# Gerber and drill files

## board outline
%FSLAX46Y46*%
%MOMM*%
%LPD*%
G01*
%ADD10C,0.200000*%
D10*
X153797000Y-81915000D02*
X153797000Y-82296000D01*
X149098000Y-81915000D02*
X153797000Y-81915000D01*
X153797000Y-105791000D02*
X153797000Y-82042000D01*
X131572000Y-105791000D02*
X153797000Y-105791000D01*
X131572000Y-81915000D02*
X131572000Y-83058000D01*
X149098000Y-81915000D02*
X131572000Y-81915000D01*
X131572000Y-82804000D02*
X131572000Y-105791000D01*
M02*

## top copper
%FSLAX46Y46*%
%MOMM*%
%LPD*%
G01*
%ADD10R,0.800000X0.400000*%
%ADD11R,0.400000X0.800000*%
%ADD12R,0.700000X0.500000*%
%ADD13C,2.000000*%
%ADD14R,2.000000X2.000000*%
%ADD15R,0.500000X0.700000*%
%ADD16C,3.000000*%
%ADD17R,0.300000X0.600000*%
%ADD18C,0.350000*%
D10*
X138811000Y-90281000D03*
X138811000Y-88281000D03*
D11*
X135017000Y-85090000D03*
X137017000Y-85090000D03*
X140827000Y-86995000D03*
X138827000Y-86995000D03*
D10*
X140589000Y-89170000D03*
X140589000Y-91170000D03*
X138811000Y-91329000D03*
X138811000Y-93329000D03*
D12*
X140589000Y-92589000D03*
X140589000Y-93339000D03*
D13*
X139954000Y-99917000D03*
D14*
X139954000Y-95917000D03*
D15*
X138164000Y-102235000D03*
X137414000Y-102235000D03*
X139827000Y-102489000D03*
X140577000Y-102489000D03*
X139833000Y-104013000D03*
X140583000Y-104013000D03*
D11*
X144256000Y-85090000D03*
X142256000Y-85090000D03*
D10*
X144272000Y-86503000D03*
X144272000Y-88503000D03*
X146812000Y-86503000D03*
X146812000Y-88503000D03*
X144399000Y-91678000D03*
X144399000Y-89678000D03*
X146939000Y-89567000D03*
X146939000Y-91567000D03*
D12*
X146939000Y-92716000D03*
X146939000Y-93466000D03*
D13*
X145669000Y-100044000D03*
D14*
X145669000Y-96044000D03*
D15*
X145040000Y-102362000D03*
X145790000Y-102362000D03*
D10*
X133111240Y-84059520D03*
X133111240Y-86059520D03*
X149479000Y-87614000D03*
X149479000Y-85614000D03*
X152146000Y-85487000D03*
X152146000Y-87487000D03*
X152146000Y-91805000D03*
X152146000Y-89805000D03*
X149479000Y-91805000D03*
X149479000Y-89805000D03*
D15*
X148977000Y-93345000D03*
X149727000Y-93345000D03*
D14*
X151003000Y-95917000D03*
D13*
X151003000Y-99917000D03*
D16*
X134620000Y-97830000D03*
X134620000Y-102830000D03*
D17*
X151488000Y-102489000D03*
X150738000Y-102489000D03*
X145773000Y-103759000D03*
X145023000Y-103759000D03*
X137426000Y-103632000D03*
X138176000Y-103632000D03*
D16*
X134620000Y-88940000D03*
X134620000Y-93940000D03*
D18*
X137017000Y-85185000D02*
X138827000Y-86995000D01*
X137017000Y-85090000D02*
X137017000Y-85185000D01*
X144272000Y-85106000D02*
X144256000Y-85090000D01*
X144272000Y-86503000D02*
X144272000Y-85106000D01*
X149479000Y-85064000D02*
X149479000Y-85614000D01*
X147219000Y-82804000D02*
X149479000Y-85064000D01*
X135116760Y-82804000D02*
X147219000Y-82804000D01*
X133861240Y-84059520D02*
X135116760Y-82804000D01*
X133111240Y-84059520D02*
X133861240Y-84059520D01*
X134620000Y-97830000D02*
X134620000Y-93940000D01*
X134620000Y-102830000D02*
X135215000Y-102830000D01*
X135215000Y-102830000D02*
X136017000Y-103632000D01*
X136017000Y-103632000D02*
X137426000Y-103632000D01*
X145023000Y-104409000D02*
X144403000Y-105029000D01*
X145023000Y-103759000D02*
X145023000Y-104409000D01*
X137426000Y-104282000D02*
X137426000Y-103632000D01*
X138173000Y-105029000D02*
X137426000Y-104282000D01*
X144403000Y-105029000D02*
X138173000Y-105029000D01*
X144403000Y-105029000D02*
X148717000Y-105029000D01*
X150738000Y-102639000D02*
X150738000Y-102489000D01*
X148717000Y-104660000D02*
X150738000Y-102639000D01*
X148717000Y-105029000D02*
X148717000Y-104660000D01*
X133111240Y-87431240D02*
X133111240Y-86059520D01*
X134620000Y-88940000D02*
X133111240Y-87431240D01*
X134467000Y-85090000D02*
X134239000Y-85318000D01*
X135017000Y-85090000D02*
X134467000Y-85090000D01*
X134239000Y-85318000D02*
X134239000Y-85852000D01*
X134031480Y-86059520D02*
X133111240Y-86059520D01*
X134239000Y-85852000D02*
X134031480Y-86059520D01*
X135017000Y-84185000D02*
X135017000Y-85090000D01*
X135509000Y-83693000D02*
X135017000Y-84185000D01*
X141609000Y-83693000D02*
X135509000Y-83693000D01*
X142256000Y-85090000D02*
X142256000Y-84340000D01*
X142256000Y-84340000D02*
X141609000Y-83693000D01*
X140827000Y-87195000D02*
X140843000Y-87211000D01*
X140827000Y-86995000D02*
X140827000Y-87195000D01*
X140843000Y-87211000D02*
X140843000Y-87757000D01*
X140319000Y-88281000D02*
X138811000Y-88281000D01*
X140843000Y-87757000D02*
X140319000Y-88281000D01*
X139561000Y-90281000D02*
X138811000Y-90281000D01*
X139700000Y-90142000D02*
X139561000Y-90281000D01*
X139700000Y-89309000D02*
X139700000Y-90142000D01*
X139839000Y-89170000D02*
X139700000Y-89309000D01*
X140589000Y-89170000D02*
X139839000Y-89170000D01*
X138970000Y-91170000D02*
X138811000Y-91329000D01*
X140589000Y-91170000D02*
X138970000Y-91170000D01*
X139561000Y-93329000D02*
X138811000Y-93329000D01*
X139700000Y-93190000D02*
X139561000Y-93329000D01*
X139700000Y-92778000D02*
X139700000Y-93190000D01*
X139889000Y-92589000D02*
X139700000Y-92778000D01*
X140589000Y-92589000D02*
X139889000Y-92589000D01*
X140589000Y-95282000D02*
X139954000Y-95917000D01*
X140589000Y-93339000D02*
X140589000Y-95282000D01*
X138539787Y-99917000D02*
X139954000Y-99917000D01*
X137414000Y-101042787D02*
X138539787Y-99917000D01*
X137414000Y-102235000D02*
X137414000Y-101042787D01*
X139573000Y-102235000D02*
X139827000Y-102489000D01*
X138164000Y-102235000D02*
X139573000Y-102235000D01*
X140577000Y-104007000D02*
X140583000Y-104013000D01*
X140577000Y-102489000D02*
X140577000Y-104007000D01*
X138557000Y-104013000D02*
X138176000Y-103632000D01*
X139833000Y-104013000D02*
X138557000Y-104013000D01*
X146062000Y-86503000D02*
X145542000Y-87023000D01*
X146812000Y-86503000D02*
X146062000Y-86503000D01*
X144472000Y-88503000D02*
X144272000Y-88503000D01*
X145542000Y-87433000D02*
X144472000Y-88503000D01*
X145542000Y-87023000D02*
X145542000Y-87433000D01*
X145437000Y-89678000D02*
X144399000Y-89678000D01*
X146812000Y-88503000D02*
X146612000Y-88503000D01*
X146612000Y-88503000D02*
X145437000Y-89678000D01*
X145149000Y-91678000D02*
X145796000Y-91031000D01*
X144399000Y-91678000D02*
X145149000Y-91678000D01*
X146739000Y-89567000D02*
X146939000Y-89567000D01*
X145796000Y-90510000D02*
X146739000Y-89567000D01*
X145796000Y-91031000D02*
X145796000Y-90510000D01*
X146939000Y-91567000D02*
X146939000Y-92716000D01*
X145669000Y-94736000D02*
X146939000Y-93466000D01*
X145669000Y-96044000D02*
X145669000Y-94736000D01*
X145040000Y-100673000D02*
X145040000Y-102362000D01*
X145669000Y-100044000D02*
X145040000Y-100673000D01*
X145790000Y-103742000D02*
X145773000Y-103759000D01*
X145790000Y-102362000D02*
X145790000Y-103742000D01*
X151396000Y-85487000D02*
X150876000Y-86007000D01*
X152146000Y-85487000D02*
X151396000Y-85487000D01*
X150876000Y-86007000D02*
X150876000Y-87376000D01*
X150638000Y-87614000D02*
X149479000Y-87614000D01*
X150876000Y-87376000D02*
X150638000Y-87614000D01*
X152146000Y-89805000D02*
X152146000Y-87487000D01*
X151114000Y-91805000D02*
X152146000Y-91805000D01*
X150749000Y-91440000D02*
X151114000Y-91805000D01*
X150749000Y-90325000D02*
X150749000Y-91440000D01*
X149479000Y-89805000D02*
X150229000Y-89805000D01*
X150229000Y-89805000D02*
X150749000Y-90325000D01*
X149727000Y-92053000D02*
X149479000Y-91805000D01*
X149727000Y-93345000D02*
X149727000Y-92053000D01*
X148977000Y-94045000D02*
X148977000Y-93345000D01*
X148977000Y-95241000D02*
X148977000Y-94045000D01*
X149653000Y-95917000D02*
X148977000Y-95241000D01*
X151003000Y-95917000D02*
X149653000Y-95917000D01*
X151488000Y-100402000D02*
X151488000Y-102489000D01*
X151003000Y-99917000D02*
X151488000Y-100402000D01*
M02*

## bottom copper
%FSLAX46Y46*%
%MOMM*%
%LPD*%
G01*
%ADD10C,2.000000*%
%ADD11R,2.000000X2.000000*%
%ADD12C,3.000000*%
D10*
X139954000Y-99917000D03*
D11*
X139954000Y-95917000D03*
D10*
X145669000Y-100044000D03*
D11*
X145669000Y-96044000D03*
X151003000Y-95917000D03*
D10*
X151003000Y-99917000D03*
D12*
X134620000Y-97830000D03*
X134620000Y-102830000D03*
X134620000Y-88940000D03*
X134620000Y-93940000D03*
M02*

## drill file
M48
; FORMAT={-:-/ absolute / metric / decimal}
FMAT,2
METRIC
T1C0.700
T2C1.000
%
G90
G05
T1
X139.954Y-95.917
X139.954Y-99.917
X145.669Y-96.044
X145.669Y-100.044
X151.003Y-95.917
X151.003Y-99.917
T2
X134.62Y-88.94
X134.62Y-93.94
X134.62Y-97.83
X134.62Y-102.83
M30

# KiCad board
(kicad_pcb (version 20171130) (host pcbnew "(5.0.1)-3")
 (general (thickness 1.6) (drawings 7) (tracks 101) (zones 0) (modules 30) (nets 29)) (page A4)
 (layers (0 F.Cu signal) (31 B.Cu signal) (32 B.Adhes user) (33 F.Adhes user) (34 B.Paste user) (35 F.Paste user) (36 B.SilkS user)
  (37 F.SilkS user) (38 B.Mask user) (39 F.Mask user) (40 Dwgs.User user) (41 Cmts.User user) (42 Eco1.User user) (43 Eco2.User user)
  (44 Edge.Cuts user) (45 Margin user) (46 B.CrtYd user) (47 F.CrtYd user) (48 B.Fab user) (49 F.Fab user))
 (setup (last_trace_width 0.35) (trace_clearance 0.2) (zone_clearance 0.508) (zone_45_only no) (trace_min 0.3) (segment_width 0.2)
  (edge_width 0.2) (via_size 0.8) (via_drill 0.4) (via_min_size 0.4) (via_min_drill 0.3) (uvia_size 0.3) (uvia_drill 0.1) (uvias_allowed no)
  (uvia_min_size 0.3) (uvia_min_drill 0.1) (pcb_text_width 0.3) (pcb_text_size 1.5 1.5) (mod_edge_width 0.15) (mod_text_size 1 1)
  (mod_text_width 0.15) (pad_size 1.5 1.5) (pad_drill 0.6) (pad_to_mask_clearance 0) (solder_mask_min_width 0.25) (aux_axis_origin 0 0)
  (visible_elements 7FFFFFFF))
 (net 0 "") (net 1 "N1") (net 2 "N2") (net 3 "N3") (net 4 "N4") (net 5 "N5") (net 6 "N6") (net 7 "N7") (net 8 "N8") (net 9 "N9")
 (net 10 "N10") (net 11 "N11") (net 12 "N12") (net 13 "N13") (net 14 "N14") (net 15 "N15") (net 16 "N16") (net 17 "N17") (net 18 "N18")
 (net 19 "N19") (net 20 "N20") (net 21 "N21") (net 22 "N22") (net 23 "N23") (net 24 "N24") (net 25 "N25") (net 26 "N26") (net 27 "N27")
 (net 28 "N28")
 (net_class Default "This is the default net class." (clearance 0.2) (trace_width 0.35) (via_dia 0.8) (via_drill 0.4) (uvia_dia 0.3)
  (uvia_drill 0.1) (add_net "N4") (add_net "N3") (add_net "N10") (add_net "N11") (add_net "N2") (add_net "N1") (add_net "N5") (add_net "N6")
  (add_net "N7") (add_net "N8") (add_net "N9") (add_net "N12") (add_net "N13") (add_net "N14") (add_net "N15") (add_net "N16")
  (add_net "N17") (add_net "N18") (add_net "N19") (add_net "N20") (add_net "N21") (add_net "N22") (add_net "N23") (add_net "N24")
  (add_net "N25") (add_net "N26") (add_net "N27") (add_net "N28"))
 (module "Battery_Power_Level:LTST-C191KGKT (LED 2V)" (layer F.Cu) (at 138.811 89.281 180)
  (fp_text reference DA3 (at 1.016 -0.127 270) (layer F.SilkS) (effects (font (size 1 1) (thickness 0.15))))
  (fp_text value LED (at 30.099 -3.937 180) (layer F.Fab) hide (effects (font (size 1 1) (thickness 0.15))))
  (pad 1 smd rect (at 0 -1 180) (size 0.8 0.4) (layers F.Cu F.Paste F.Mask) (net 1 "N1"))
  (pad 2 smd rect (at 0 1 180) (size 0.8 0.4) (layers F.Cu F.Paste F.Mask) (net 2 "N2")))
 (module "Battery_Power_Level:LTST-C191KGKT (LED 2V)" (layer F.Cu) (at 136.017 85.09 270)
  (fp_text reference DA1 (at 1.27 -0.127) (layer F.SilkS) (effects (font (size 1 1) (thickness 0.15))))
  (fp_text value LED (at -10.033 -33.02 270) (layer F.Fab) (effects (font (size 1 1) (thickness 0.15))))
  (pad 2 smd rect (at 0 1 270) (size 0.8 0.4) (layers F.Cu F.Paste F.Mask) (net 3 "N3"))
  (pad 1 smd rect (at 0 -1 270) (size 0.8 0.4) (layers F.Cu F.Paste F.Mask) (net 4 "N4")))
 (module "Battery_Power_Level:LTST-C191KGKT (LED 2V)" (layer F.Cu) (at 139.827 86.995 270)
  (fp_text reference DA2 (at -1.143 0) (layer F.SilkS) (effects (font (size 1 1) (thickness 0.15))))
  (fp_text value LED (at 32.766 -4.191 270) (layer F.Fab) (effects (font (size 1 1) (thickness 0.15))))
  (pad 1 smd rect (at 0 -1 270) (size 0.8 0.4) (layers F.Cu F.Paste F.Mask) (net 2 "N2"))
  (pad 2 smd rect (at 0 1 270) (size 0.8 0.4) (layers F.Cu F.Paste F.Mask) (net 4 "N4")))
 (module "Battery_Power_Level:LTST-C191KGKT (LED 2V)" (layer F.Cu) (at 140.589 90.17 180)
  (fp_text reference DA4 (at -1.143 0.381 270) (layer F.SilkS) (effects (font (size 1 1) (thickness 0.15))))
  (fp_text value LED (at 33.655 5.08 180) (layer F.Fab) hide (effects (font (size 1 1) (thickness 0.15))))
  (pad 2 smd rect (at 0 1 180) (size 0.8 0.4) (layers F.Cu F.Paste F.Mask) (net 1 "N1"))
  (pad 1 smd rect (at 0 -1 180) (size 0.8 0.4) (layers F.Cu F.Paste F.Mask) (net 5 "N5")))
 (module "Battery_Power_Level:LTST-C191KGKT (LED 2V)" (layer F.Cu) (at 138.811 92.329 180)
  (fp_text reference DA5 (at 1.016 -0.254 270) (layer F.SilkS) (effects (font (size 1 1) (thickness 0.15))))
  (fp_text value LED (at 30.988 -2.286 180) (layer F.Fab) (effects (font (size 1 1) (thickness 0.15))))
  (pad 2 smd rect (at 0 1 180) (size 0.8 0.4) (layers F.Cu F.Paste F.Mask) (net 5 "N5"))
  (pad 1 smd rect (at 0 -1 180) (size 0.8 0.4) (layers F.Cu F.Paste F.Mask) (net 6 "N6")))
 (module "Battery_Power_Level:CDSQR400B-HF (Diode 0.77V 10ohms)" (layer F.Cu) (at 140.589 92.964 270)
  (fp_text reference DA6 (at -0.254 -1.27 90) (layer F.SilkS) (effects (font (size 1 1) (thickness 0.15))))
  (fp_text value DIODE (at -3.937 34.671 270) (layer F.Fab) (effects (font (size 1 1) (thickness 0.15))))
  (pad 1 smd rect (at -0.375 0 270) (size 0.5 0.7) (layers F.Cu F.Paste F.Mask) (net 6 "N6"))
  (pad 2 smd rect (at 0.375 0 270) (size 0.5 0.7) (layers F.Cu F.Paste F.Mask) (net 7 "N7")))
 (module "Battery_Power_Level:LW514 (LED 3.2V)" (layer F.Cu) (at 139.954 97.917 270)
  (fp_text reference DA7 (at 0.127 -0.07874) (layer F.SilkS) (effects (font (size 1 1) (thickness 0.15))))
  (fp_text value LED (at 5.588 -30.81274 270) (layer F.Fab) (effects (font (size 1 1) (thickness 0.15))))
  (pad 1 thru_hole circle (at 2 0 270) (size 2 2) (drill 0.7) (layers *.Cu *.Mask) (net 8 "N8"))
  (pad 2 thru_hole rect (at -2 0 270) (size 2 2) (drill 0.7) (layers *.Cu *.Mask) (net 7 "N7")))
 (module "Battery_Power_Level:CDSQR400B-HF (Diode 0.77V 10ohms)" (layer F.Cu) (at 137.789 102.235)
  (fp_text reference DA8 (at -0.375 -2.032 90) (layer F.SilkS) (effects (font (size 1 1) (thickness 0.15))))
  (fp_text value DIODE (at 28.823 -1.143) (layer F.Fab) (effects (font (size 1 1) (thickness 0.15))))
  (pad 2 smd rect (at 0.375 0) (size 0.5 0.7) (layers F.Cu F.Paste F.Mask) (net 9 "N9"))
  (pad 1 smd rect (at -0.375 0) (size 0.5 0.7) (layers F.Cu F.Paste F.Mask) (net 8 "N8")))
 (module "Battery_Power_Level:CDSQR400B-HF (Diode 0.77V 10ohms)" (layer F.Cu) (at 140.202 102.489)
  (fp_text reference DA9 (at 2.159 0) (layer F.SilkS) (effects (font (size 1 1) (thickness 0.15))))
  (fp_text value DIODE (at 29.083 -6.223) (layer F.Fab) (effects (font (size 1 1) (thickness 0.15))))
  (pad 1 smd rect (at -0.375 0) (size 0.5 0.7) (layers F.Cu F.Paste F.Mask) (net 9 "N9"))
  (pad 2 smd rect (at 0.375 0) (size 0.5 0.7) (layers F.Cu F.Paste F.Mask) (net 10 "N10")))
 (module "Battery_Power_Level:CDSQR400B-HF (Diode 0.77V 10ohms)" (layer F.Cu) (at 140.208 104.013 180)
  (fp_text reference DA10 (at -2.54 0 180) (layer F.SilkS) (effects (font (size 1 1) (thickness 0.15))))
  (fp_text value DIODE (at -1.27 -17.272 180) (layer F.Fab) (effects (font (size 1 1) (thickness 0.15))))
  (pad 2 smd rect (at 0.375 0 180) (size 0.5 0.7) (layers F.Cu F.Paste F.Mask) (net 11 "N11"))
  (pad 1 smd rect (at -0.375 0 180) (size 0.5 0.7) (layers F.Cu F.Paste F.Mask) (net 10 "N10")))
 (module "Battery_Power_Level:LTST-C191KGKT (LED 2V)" (layer F.Cu) (at 143.256 85.09 270)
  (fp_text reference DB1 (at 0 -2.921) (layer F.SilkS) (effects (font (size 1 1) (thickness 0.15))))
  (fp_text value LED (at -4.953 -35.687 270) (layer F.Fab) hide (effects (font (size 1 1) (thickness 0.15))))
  (pad 1 smd rect (at 0 -1 270) (size 0.8 0.4) (layers F.Cu F.Paste F.Mask) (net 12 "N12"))
  (pad 2 smd rect (at 0 1 270) (size 0.8 0.4) (layers F.Cu F.Paste F.Mask) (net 3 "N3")))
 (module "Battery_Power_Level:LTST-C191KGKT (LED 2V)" (layer F.Cu) (at 144.272 87.503 180)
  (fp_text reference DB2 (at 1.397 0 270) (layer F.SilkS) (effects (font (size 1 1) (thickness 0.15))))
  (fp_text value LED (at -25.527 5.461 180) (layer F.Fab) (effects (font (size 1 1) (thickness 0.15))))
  (pad 2 smd rect (at 0 1 180) (size 0.8 0.4) (layers F.Cu F.Paste F.Mask) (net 12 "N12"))
  (pad 1 smd rect (at 0 -1 180) (size 0.8 0.4) (layers F.Cu F.Paste F.Mask) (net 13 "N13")))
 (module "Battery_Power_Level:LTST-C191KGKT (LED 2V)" (layer F.Cu) (at 146.812 87.503 180)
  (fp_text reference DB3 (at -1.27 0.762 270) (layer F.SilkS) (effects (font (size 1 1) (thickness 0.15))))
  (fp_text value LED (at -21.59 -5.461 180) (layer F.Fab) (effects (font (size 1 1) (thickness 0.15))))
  (pad 2 smd rect (at 0 1 180) (size 0.8 0.4) (layers F.Cu F.Paste F.Mask) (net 13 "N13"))
  (pad 1 smd rect (at 0 -1 180) (size 0.8 0.4) (layers F.Cu F.Paste F.Mask) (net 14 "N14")))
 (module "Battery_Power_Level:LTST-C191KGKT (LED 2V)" (layer F.Cu) (at 144.399 90.678 180)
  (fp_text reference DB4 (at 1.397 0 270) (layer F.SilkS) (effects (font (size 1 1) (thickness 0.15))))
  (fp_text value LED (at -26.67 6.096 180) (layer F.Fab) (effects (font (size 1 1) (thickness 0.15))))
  (pad 1 smd rect (at 0 -1 180) (size 0.8 0.4) (layers F.Cu F.Paste F.Mask) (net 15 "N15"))
  (pad 2 smd rect (at 0 1 180) (size 0.8 0.4) (layers F.Cu F.Paste F.Mask) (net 14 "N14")))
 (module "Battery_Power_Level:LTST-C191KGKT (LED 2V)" (layer F.Cu) (at 146.939 90.567 180)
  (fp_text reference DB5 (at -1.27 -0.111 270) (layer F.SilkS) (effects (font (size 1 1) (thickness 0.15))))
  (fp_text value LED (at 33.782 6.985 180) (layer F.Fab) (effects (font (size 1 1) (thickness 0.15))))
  (pad 2 smd rect (at 0 1 180) (size 0.8 0.4) (layers F.Cu F.Paste F.Mask) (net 15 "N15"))
  (pad 1 smd rect (at 0 -1 180) (size 0.8 0.4) (layers F.Cu F.Paste F.Mask) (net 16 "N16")))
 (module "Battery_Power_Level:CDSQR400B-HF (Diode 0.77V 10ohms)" (layer F.Cu) (at 146.939 93.091 270)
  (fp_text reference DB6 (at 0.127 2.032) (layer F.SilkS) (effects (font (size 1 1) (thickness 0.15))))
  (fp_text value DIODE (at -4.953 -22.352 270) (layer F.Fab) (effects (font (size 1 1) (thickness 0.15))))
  (pad 1 smd rect (at -0.375 0 270) (size 0.5 0.7) (layers F.Cu F.Paste F.Mask) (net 16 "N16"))
  (pad 2 smd rect (at 0.375 0 270) (size 0.5 0.7) (layers F.Cu F.Paste F.Mask) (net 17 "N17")))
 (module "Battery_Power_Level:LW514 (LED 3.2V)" (layer F.Cu) (at 145.669 98.044 270)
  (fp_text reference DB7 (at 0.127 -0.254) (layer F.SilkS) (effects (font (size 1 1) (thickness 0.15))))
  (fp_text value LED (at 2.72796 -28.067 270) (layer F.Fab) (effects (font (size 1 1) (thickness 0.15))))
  (pad 1 thru_hole circle (at 2 0 270) (size 2 2) (drill 0.7) (layers *.Cu *.Mask) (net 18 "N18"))
  (pad 2 thru_hole rect (at -2 0 270) (size 2 2) (drill 0.7) (layers *.Cu *.Mask) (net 17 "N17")))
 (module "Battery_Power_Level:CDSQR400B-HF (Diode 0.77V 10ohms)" (layer F.Cu) (at 145.415 102.362)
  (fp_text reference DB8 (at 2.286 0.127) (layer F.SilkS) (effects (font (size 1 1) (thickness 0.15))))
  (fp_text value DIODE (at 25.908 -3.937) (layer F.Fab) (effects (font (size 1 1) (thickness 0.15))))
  (pad 1 smd rect (at -0.375 0) (size 0.5 0.7) (layers F.Cu F.Paste F.Mask) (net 18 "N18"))
  (pad 2 smd rect (at 0.375 0) (size 0.5 0.7) (layers F.Cu F.Paste F.Mask) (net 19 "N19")))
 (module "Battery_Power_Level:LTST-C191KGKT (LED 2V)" (layer F.Cu) (at 133.11124 85.05952)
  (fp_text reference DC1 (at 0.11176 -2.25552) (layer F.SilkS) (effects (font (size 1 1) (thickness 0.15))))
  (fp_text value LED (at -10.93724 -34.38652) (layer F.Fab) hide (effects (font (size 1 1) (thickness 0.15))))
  (pad 1 smd rect (at 0 -1) (size 0.8 0.4) (layers F.Cu F.Paste F.Mask) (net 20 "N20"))
  (pad 2 smd rect (at 0 1) (size 0.8 0.4) (layers F.Cu F.Paste F.Mask) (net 3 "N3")))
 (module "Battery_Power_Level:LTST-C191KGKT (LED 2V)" (layer F.Cu) (at 149.479 86.614 180)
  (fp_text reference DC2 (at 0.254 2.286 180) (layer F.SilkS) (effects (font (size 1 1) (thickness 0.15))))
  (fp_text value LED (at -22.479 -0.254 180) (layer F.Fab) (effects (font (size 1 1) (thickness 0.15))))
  (pad 1 smd rect (at 0 -1 180) (size 0.8 0.4) (layers F.Cu F.Paste F.Mask) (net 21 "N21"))
  (pad 2 smd rect (at 0 1 180) (size 0.8 0.4) (layers F.Cu F.Paste F.Mask) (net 20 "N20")))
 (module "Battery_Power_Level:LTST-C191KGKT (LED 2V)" (layer F.Cu) (at 152.146 86.487 180)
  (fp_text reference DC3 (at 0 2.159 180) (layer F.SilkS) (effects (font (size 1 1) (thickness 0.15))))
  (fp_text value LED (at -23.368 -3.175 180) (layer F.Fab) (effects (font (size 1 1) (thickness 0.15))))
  (pad 2 smd rect (at 0 1 180) (size 0.8 0.4) (layers F.Cu F.Paste F.Mask) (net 21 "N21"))
  (pad 1 smd rect (at 0 -1 180) (size 0.8 0.4) (layers F.Cu F.Paste F.Mask) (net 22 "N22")))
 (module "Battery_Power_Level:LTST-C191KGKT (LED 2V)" (layer F.Cu) (at 152.146 90.805 180)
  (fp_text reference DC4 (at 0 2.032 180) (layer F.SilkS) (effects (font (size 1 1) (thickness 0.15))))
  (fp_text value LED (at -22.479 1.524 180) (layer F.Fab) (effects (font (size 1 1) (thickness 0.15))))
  (pad 1 smd rect (at 0 -1 180) (size 0.8 0.4) (layers F.Cu F.Paste F.Mask) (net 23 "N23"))
  (pad 2 smd rect (at 0 1 180) (size 0.8 0.4) (layers F.Cu F.Paste F.Mask) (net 22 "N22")))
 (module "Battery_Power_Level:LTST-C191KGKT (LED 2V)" (layer F.Cu) (at 149.479 90.805 180)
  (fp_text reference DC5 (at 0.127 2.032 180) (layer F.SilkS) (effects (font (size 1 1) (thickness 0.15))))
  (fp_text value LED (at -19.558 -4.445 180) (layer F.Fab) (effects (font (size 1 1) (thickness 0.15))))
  (pad 1 smd rect (at 0 -1 180) (size 0.8 0.4) (layers F.Cu F.Paste F.Mask) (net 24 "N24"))
  (pad 2 smd rect (at 0 1 180) (size 0.8 0.4) (layers F.Cu F.Paste F.Mask) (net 23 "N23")))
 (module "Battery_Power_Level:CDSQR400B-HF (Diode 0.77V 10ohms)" (layer F.Cu) (at 149.352 93.345 180)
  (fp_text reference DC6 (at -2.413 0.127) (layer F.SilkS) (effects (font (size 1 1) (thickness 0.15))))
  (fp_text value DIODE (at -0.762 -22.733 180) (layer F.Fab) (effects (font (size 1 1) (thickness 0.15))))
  (pad 2 smd rect (at 0.375 0 180) (size 0.5 0.7) (layers F.Cu F.Paste F.Mask) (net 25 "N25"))
  (pad 1 smd rect (at -0.375 0 180) (size 0.5 0.7) (layers F.Cu F.Paste F.Mask) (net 24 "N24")))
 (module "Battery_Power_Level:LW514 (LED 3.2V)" (layer F.Cu) (at 151.003 97.917 270)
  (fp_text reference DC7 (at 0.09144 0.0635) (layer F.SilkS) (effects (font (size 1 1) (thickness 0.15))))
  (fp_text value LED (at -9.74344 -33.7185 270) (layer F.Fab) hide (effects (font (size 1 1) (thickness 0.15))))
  (pad 2 thru_hole rect (at -2 0 270) (size 2 2) (drill 0.7) (layers *.Cu *.Mask) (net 25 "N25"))
  (pad 1 thru_hole circle (at 2 0 270) (size 2 2) (drill 0.7) (layers *.Cu *.Mask) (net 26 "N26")))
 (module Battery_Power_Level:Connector (layer F.Cu) (at 134.62 100.33 270)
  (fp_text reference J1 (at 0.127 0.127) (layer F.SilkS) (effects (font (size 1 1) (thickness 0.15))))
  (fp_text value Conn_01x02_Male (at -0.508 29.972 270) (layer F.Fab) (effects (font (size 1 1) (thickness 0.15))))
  (pad 1 thru_hole circle (at -2.5 0 270) (size 3 3) (drill 1) (layers *.Cu *.Mask) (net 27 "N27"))
  (pad 2 thru_hole circle (at 2.5 0 270) (size 3 3) (drill 1) (layers *.Cu *.Mask) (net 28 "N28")))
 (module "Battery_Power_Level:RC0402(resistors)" (layer F.Cu) (at 151.638 102.489 180)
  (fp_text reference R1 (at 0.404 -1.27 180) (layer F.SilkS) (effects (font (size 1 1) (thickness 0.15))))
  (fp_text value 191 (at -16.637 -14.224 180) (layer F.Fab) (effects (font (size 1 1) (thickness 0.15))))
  (pad 1 smd rect (at 0.15 0 180) (size 0.3 0.6) (layers F.Cu F.Paste F.Mask) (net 26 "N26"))
  (pad 2 smd rect (at 0.9 0 180) (size 0.3 0.6) (layers F.Cu F.Paste F.Mask) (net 28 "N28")))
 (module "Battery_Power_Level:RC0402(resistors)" (layer F.Cu) (at 145.923 103.759 180)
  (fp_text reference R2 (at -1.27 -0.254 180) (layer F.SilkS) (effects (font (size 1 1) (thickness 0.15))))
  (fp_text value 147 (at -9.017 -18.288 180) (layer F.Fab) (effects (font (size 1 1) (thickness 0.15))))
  (pad 1 smd rect (at 0.15 0 180) (size 0.3 0.6) (layers F.Cu F.Paste F.Mask) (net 19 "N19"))
  (pad 2 smd rect (at 0.9 0 180) (size 0.3 0.6) (layers F.Cu F.Paste F.Mask) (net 28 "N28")))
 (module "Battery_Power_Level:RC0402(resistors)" (layer F.Cu) (at 138.326 103.632 180)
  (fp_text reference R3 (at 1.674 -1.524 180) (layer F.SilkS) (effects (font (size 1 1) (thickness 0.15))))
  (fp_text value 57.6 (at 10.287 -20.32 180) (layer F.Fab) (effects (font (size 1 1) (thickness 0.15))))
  (pad 2 smd rect (at 0.9 0 180) (size 0.3 0.6) (layers F.Cu F.Paste F.Mask) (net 28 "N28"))
  (pad 1 smd rect (at 0.15 0 180) (size 0.3 0.6) (layers F.Cu F.Paste F.Mask) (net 11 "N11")))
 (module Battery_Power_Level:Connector (layer F.Cu) (at 134.62 91.44 90)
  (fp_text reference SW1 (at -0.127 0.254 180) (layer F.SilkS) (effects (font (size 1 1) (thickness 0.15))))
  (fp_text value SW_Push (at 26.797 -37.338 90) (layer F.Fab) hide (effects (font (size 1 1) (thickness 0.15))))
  (pad 2 thru_hole circle (at 2.5 0 90) (size 3 3) (drill 1) (layers *.Cu *.Mask) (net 3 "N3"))
  (pad 1 thru_hole circle (at -2.5 0 90) (size 3 3) (drill 1) (layers *.Cu *.Mask) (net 27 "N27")))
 (gr_line (start 153.797 81.915) (end 153.797 82.296) (layer Edge.Cuts) (width 0.2))
 (gr_line (start 149.098 81.915) (end 153.797 81.915) (layer Edge.Cuts) (width 0.2))
 (gr_line (start 153.797 105.791) (end 153.797 82.042) (layer Edge.Cuts) (width 0.2))
 (gr_line (start 131.572 105.791) (end 153.797 105.791) (layer Edge.Cuts) (width 0.2))
 (gr_line (start 131.572 81.915) (end 131.572 83.058) (layer Edge.Cuts) (width 0.2))
 (gr_line (start 149.098 81.915) (end 131.572 81.915) (layer Edge.Cuts) (width 0.2))
 (gr_line (start 131.572 82.804) (end 131.572 105.791) (layer Edge.Cuts) (width 0.2))
 (segment (start 137.017 85.185) (end 138.827 86.995) (width 0.35) (layer F.Cu) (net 4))
 (segment (start 137.017 85.09) (end 137.017 85.185) (width 0.35) (layer F.Cu) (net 4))
 (segment (start 144.272 85.106) (end 144.256 85.09) (width 0.35) (layer F.Cu) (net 12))
 (segment (start 144.272 86.503) (end 144.272 85.106) (width 0.35) (layer F.Cu) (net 12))
 (segment (start 149.479 85.064) (end 149.479 85.614) (width 0.35) (layer F.Cu) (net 20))
 (segment (start 147.219 82.804) (end 149.479 85.064) (width 0.35) (layer F.Cu) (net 20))
 (segment (start 135.11676 82.804) (end 147.219 82.804) (width 0.35) (layer F.Cu) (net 20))
 (segment (start 133.86124 84.05952) (end 135.11676 82.804) (width 0.35) (layer F.Cu) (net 20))
 (segment (start 133.11124 84.05952) (end 133.86124 84.05952) (width 0.35) (layer F.Cu) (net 20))
 (segment (start 134.62 97.83) (end 134.62 93.94) (width 0.35) (layer F.Cu) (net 27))
 (segment (start 134.62 102.83) (end 135.215 102.83) (width 0.35) (layer F.Cu) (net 28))
 (segment (start 135.215 102.83) (end 136.017 103.632) (width 0.35) (layer F.Cu) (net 28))
 (segment (start 136.017 103.632) (end 137.426 103.632) (width 0.35) (layer F.Cu) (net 28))
 (segment (start 145.023 104.409) (end 144.403 105.029) (width 0.35) (layer F.Cu) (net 28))
 (segment (start 145.023 103.759) (end 145.023 104.409) (width 0.35) (layer F.Cu) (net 28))
 (segment (start 137.426 104.282) (end 137.426 103.632) (width 0.35) (layer F.Cu) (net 28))
 (segment (start 138.173 105.029) (end 137.426 104.282) (width 0.35) (layer F.Cu) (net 28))
 (segment (start 144.403 105.029) (end 138.173 105.029) (width 0.35) (layer F.Cu) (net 28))
 (segment (start 144.403 105.029) (end 148.717 105.029) (width 0.35) (layer F.Cu) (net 28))
 (segment (start 150.738 102.639) (end 150.738 102.489) (width 0.35) (layer F.Cu) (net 28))
 (segment (start 148.717 104.66) (end 150.738 102.639) (width 0.35) (layer F.Cu) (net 28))
 (segment (start 148.717 105.029) (end 148.717 104.66) (width 0.35) (layer F.Cu) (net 28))
 (segment (start 133.11124 87.43124) (end 133.11124 86.05952) (width 0.35) (layer F.Cu) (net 3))
 (segment (start 134.62 88.94) (end 133.11124 87.43124) (width 0.35) (layer F.Cu) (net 3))
 (segment (start 134.467 85.09) (end 134.239 85.318) (width 0.35) (layer F.Cu) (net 3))
 (segment (start 135.017 85.09) (end 134.467 85.09) (width 0.35) (layer F.Cu) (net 3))
 (segment (start 134.239 85.318) (end 134.239 85.852) (width 0.35) (layer F.Cu) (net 3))
 (segment (start 134.03148 86.05952) (end 133.11124 86.05952) (width 0.35) (layer F.Cu) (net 3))
 (segment (start 134.239 85.852) (end 134.03148 86.05952) (width 0.35) (layer F.Cu) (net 3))
 (segment (start 135.017 84.185) (end 135.017 85.09) (width 0.35) (layer F.Cu) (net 3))
 (segment (start 135.509 83.693) (end 135.017 84.185) (width 0.35) (layer F.Cu) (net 3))
 (segment (start 141.609 83.693) (end 135.509 83.693) (width 0.35) (layer F.Cu) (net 3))
 (segment (start 142.256 85.09) (end 142.256 84.34) (width 0.35) (layer F.Cu) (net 3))
 (segment (start 142.256 84.34) (end 141.609 83.693) (width 0.35) (layer F.Cu) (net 3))
 (segment (start 140.827 87.195) (end 140.843 87.211) (width 0.35) (layer F.Cu) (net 2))
 (segment (start 140.827 86.995) (end 140.827 87.195) (width 0.35) (layer F.Cu) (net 2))
 (segment (start 140.843 87.211) (end 140.843 87.757) (width 0.35) (layer F.Cu) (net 2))
 (segment (start 140.319 88.281) (end 138.811 88.281) (width 0.35) (layer F.Cu) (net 2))
 (segment (start 140.843 87.757) (end 140.319 88.281) (width 0.35) (layer F.Cu) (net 2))
 (segment (start 139.561 90.281) (end 138.811 90.281) (width 0.35) (layer F.Cu) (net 1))
 (segment (start 139.7 90.142) (end 139.561 90.281) (width 0.35) (layer F.Cu) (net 1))
 (segment (start 139.7 89.309) (end 139.7 90.142) (width 0.35) (layer F.Cu) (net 1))
 (segment (start 139.839 89.17) (end 139.7 89.309) (width 0.35) (layer F.Cu) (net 1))
 (segment (start 140.589 89.17) (end 139.839 89.17) (width 0.35) (layer F.Cu) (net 1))
 (segment (start 138.97 91.17) (end 138.811 91.329) (width 0.35) (layer F.Cu) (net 5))
 (segment (start 140.589 91.17) (end 138.97 91.17) (width 0.35) (layer F.Cu) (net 5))
 (segment (start 139.561 93.329) (end 138.811 93.329) (width 0.35) (layer F.Cu) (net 6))
 (segment (start 139.7 93.19) (end 139.561 93.329) (width 0.35) (layer F.Cu) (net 6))
 (segment (start 139.7 92.778) (end 139.7 93.19) (width 0.35) (layer F.Cu) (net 6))
 (segment (start 139.889 92.589) (end 139.7 92.778) (width 0.35) (layer F.Cu) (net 6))
 (segment (start 140.589 92.589) (end 139.889 92.589) (width 0.35) (layer F.Cu) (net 6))
 (segment (start 140.589 95.282) (end 139.954 95.917) (width 0.35) (layer F.Cu) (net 7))
 (segment (start 140.589 93.339) (end 140.589 95.282) (width 0.35) (layer F.Cu) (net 7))
 (segment (start 138.539787 99.917) (end 139.954 99.917) (width 0.35) (layer F.Cu) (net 8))
 (segment (start 137.414 101.042787) (end 138.539787 99.917) (width 0.35) (layer F.Cu) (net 8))
 (segment (start 137.414 102.235) (end 137.414 101.042787) (width 0.35) (layer F.Cu) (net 8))
 (segment (start 139.573 102.235) (end 139.827 102.489) (width 0.35) (layer F.Cu) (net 9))
 (segment (start 138.164 102.235) (end 139.573 102.235) (width 0.35) (layer F.Cu) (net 9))
 (segment (start 140.577 104.007) (end 140.583 104.013) (width 0.35) (layer F.Cu) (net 10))
 (segment (start 140.577 102.489) (end 140.577 104.007) (width 0.35) (layer F.Cu) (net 10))
 (segment (start 138.557 104.013) (end 138.176 103.632) (width 0.35) (layer F.Cu) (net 11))
 (segment (start 139.833 104.013) (end 138.557 104.013) (width 0.35) (layer F.Cu) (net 11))
 (segment (start 146.062 86.503) (end 145.542 87.023) (width 0.35) (layer F.Cu) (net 13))
 (segment (start 146.812 86.503) (end 146.062 86.503) (width 0.35) (layer F.Cu) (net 13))
 (segment (start 144.472 88.503) (end 144.272 88.503) (width 0.35) (layer F.Cu) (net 13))
 (segment (start 145.542 87.433) (end 144.472 88.503) (width 0.35) (layer F.Cu) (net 13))
 (segment (start 145.542 87.023) (end 145.542 87.433) (width 0.35) (layer F.Cu) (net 13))
 (segment (start 145.437 89.678) (end 144.399 89.678) (width 0.35) (layer F.Cu) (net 14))
 (segment (start 146.812 88.503) (end 146.612 88.503) (width 0.35) (layer F.Cu) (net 14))
 (segment (start 146.612 88.503) (end 145.437 89.678) (width 0.35) (layer F.Cu) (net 14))
 (segment (start 145.149 91.678) (end 145.796 91.031) (width 0.35) (layer F.Cu) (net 15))
 (segment (start 144.399 91.678) (end 145.149 91.678) (width 0.35) (layer F.Cu) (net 15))
 (segment (start 146.739 89.567) (end 146.939 89.567) (width 0.35) (layer F.Cu) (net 15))
 (segment (start 145.796 90.51) (end 146.739 89.567) (width 0.35) (layer F.Cu) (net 15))
 (segment (start 145.796 91.031) (end 145.796 90.51) (width 0.35) (layer F.Cu) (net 15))
 (segment (start 146.939 91.567) (end 146.939 92.716) (width 0.35) (layer F.Cu) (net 16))
 (segment (start 145.669 94.736) (end 146.939 93.466) (width 0.35) (layer F.Cu) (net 17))
 (segment (start 145.669 96.044) (end 145.669 94.736) (width 0.35) (layer F.Cu) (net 17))
 (segment (start 145.04 100.673) (end 145.04 102.362) (width 0.35) (layer F.Cu) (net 18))
 (segment (start 145.669 100.044) (end 145.04 100.673) (width 0.35) (layer F.Cu) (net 18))
 (segment (start 145.79 103.742) (end 145.773 103.759) (width 0.35) (layer F.Cu) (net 19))
 (segment (start 145.79 102.362) (end 145.79 103.742) (width 0.35) (layer F.Cu) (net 19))
 (segment (start 151.396 85.487) (end 150.876 86.007) (width 0.35) (layer F.Cu) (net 21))
 (segment (start 152.146 85.487) (end 151.396 85.487) (width 0.35) (layer F.Cu) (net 21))
 (segment (start 150.876 86.007) (end 150.876 87.376) (width 0.35) (layer F.Cu) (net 21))
 (segment (start 150.638 87.614) (end 149.479 87.614) (width 0.35) (layer F.Cu) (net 21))
 (segment (start 150.876 87.376) (end 150.638 87.614) (width 0.35) (layer F.Cu) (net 21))
 (segment (start 152.146 89.805) (end 152.146 87.487) (width 0.35) (layer F.Cu) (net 22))
 (segment (start 151.114 91.805) (end 152.146 91.805) (width 0.35) (layer F.Cu) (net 23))
 (segment (start 150.749 91.44) (end 151.114 91.805) (width 0.35) (layer F.Cu) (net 23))
 (segment (start 150.749 90.325) (end 150.749 91.44) (width 0.35) (layer F.Cu) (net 23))
 (segment (start 149.479 89.805) (end 150.229 89.805) (width 0.35) (layer F.Cu) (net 23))
 (segment (start 150.229 89.805) (end 150.749 90.325) (width 0.35) (layer F.Cu) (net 23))
 (segment (start 149.727 92.053) (end 149.479 91.805) (width 0.35) (layer F.Cu) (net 24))
 (segment (start 149.727 93.345) (end 149.727 92.053) (width 0.35) (layer F.Cu) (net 24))
 (segment (start 148.977 94.045) (end 148.977 93.345) (width 0.35) (layer F.Cu) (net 25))
 (segment (start 148.977 95.241) (end 148.977 94.045) (width 0.35) (layer F.Cu) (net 25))
 (segment (start 149.653 95.917) (end 148.977 95.241) (width 0.35) (layer F.Cu) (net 25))
 (segment (start 151.003 95.917) (end 149.653 95.917) (width 0.35) (layer F.Cu) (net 25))
 (segment (start 151.488 100.402) (end 151.488 102.489) (width 0.35) (layer F.Cu) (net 26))
 (segment (start 151.003 99.917) (end 151.488 100.402) (width 0.35) (layer F.Cu) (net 26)))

